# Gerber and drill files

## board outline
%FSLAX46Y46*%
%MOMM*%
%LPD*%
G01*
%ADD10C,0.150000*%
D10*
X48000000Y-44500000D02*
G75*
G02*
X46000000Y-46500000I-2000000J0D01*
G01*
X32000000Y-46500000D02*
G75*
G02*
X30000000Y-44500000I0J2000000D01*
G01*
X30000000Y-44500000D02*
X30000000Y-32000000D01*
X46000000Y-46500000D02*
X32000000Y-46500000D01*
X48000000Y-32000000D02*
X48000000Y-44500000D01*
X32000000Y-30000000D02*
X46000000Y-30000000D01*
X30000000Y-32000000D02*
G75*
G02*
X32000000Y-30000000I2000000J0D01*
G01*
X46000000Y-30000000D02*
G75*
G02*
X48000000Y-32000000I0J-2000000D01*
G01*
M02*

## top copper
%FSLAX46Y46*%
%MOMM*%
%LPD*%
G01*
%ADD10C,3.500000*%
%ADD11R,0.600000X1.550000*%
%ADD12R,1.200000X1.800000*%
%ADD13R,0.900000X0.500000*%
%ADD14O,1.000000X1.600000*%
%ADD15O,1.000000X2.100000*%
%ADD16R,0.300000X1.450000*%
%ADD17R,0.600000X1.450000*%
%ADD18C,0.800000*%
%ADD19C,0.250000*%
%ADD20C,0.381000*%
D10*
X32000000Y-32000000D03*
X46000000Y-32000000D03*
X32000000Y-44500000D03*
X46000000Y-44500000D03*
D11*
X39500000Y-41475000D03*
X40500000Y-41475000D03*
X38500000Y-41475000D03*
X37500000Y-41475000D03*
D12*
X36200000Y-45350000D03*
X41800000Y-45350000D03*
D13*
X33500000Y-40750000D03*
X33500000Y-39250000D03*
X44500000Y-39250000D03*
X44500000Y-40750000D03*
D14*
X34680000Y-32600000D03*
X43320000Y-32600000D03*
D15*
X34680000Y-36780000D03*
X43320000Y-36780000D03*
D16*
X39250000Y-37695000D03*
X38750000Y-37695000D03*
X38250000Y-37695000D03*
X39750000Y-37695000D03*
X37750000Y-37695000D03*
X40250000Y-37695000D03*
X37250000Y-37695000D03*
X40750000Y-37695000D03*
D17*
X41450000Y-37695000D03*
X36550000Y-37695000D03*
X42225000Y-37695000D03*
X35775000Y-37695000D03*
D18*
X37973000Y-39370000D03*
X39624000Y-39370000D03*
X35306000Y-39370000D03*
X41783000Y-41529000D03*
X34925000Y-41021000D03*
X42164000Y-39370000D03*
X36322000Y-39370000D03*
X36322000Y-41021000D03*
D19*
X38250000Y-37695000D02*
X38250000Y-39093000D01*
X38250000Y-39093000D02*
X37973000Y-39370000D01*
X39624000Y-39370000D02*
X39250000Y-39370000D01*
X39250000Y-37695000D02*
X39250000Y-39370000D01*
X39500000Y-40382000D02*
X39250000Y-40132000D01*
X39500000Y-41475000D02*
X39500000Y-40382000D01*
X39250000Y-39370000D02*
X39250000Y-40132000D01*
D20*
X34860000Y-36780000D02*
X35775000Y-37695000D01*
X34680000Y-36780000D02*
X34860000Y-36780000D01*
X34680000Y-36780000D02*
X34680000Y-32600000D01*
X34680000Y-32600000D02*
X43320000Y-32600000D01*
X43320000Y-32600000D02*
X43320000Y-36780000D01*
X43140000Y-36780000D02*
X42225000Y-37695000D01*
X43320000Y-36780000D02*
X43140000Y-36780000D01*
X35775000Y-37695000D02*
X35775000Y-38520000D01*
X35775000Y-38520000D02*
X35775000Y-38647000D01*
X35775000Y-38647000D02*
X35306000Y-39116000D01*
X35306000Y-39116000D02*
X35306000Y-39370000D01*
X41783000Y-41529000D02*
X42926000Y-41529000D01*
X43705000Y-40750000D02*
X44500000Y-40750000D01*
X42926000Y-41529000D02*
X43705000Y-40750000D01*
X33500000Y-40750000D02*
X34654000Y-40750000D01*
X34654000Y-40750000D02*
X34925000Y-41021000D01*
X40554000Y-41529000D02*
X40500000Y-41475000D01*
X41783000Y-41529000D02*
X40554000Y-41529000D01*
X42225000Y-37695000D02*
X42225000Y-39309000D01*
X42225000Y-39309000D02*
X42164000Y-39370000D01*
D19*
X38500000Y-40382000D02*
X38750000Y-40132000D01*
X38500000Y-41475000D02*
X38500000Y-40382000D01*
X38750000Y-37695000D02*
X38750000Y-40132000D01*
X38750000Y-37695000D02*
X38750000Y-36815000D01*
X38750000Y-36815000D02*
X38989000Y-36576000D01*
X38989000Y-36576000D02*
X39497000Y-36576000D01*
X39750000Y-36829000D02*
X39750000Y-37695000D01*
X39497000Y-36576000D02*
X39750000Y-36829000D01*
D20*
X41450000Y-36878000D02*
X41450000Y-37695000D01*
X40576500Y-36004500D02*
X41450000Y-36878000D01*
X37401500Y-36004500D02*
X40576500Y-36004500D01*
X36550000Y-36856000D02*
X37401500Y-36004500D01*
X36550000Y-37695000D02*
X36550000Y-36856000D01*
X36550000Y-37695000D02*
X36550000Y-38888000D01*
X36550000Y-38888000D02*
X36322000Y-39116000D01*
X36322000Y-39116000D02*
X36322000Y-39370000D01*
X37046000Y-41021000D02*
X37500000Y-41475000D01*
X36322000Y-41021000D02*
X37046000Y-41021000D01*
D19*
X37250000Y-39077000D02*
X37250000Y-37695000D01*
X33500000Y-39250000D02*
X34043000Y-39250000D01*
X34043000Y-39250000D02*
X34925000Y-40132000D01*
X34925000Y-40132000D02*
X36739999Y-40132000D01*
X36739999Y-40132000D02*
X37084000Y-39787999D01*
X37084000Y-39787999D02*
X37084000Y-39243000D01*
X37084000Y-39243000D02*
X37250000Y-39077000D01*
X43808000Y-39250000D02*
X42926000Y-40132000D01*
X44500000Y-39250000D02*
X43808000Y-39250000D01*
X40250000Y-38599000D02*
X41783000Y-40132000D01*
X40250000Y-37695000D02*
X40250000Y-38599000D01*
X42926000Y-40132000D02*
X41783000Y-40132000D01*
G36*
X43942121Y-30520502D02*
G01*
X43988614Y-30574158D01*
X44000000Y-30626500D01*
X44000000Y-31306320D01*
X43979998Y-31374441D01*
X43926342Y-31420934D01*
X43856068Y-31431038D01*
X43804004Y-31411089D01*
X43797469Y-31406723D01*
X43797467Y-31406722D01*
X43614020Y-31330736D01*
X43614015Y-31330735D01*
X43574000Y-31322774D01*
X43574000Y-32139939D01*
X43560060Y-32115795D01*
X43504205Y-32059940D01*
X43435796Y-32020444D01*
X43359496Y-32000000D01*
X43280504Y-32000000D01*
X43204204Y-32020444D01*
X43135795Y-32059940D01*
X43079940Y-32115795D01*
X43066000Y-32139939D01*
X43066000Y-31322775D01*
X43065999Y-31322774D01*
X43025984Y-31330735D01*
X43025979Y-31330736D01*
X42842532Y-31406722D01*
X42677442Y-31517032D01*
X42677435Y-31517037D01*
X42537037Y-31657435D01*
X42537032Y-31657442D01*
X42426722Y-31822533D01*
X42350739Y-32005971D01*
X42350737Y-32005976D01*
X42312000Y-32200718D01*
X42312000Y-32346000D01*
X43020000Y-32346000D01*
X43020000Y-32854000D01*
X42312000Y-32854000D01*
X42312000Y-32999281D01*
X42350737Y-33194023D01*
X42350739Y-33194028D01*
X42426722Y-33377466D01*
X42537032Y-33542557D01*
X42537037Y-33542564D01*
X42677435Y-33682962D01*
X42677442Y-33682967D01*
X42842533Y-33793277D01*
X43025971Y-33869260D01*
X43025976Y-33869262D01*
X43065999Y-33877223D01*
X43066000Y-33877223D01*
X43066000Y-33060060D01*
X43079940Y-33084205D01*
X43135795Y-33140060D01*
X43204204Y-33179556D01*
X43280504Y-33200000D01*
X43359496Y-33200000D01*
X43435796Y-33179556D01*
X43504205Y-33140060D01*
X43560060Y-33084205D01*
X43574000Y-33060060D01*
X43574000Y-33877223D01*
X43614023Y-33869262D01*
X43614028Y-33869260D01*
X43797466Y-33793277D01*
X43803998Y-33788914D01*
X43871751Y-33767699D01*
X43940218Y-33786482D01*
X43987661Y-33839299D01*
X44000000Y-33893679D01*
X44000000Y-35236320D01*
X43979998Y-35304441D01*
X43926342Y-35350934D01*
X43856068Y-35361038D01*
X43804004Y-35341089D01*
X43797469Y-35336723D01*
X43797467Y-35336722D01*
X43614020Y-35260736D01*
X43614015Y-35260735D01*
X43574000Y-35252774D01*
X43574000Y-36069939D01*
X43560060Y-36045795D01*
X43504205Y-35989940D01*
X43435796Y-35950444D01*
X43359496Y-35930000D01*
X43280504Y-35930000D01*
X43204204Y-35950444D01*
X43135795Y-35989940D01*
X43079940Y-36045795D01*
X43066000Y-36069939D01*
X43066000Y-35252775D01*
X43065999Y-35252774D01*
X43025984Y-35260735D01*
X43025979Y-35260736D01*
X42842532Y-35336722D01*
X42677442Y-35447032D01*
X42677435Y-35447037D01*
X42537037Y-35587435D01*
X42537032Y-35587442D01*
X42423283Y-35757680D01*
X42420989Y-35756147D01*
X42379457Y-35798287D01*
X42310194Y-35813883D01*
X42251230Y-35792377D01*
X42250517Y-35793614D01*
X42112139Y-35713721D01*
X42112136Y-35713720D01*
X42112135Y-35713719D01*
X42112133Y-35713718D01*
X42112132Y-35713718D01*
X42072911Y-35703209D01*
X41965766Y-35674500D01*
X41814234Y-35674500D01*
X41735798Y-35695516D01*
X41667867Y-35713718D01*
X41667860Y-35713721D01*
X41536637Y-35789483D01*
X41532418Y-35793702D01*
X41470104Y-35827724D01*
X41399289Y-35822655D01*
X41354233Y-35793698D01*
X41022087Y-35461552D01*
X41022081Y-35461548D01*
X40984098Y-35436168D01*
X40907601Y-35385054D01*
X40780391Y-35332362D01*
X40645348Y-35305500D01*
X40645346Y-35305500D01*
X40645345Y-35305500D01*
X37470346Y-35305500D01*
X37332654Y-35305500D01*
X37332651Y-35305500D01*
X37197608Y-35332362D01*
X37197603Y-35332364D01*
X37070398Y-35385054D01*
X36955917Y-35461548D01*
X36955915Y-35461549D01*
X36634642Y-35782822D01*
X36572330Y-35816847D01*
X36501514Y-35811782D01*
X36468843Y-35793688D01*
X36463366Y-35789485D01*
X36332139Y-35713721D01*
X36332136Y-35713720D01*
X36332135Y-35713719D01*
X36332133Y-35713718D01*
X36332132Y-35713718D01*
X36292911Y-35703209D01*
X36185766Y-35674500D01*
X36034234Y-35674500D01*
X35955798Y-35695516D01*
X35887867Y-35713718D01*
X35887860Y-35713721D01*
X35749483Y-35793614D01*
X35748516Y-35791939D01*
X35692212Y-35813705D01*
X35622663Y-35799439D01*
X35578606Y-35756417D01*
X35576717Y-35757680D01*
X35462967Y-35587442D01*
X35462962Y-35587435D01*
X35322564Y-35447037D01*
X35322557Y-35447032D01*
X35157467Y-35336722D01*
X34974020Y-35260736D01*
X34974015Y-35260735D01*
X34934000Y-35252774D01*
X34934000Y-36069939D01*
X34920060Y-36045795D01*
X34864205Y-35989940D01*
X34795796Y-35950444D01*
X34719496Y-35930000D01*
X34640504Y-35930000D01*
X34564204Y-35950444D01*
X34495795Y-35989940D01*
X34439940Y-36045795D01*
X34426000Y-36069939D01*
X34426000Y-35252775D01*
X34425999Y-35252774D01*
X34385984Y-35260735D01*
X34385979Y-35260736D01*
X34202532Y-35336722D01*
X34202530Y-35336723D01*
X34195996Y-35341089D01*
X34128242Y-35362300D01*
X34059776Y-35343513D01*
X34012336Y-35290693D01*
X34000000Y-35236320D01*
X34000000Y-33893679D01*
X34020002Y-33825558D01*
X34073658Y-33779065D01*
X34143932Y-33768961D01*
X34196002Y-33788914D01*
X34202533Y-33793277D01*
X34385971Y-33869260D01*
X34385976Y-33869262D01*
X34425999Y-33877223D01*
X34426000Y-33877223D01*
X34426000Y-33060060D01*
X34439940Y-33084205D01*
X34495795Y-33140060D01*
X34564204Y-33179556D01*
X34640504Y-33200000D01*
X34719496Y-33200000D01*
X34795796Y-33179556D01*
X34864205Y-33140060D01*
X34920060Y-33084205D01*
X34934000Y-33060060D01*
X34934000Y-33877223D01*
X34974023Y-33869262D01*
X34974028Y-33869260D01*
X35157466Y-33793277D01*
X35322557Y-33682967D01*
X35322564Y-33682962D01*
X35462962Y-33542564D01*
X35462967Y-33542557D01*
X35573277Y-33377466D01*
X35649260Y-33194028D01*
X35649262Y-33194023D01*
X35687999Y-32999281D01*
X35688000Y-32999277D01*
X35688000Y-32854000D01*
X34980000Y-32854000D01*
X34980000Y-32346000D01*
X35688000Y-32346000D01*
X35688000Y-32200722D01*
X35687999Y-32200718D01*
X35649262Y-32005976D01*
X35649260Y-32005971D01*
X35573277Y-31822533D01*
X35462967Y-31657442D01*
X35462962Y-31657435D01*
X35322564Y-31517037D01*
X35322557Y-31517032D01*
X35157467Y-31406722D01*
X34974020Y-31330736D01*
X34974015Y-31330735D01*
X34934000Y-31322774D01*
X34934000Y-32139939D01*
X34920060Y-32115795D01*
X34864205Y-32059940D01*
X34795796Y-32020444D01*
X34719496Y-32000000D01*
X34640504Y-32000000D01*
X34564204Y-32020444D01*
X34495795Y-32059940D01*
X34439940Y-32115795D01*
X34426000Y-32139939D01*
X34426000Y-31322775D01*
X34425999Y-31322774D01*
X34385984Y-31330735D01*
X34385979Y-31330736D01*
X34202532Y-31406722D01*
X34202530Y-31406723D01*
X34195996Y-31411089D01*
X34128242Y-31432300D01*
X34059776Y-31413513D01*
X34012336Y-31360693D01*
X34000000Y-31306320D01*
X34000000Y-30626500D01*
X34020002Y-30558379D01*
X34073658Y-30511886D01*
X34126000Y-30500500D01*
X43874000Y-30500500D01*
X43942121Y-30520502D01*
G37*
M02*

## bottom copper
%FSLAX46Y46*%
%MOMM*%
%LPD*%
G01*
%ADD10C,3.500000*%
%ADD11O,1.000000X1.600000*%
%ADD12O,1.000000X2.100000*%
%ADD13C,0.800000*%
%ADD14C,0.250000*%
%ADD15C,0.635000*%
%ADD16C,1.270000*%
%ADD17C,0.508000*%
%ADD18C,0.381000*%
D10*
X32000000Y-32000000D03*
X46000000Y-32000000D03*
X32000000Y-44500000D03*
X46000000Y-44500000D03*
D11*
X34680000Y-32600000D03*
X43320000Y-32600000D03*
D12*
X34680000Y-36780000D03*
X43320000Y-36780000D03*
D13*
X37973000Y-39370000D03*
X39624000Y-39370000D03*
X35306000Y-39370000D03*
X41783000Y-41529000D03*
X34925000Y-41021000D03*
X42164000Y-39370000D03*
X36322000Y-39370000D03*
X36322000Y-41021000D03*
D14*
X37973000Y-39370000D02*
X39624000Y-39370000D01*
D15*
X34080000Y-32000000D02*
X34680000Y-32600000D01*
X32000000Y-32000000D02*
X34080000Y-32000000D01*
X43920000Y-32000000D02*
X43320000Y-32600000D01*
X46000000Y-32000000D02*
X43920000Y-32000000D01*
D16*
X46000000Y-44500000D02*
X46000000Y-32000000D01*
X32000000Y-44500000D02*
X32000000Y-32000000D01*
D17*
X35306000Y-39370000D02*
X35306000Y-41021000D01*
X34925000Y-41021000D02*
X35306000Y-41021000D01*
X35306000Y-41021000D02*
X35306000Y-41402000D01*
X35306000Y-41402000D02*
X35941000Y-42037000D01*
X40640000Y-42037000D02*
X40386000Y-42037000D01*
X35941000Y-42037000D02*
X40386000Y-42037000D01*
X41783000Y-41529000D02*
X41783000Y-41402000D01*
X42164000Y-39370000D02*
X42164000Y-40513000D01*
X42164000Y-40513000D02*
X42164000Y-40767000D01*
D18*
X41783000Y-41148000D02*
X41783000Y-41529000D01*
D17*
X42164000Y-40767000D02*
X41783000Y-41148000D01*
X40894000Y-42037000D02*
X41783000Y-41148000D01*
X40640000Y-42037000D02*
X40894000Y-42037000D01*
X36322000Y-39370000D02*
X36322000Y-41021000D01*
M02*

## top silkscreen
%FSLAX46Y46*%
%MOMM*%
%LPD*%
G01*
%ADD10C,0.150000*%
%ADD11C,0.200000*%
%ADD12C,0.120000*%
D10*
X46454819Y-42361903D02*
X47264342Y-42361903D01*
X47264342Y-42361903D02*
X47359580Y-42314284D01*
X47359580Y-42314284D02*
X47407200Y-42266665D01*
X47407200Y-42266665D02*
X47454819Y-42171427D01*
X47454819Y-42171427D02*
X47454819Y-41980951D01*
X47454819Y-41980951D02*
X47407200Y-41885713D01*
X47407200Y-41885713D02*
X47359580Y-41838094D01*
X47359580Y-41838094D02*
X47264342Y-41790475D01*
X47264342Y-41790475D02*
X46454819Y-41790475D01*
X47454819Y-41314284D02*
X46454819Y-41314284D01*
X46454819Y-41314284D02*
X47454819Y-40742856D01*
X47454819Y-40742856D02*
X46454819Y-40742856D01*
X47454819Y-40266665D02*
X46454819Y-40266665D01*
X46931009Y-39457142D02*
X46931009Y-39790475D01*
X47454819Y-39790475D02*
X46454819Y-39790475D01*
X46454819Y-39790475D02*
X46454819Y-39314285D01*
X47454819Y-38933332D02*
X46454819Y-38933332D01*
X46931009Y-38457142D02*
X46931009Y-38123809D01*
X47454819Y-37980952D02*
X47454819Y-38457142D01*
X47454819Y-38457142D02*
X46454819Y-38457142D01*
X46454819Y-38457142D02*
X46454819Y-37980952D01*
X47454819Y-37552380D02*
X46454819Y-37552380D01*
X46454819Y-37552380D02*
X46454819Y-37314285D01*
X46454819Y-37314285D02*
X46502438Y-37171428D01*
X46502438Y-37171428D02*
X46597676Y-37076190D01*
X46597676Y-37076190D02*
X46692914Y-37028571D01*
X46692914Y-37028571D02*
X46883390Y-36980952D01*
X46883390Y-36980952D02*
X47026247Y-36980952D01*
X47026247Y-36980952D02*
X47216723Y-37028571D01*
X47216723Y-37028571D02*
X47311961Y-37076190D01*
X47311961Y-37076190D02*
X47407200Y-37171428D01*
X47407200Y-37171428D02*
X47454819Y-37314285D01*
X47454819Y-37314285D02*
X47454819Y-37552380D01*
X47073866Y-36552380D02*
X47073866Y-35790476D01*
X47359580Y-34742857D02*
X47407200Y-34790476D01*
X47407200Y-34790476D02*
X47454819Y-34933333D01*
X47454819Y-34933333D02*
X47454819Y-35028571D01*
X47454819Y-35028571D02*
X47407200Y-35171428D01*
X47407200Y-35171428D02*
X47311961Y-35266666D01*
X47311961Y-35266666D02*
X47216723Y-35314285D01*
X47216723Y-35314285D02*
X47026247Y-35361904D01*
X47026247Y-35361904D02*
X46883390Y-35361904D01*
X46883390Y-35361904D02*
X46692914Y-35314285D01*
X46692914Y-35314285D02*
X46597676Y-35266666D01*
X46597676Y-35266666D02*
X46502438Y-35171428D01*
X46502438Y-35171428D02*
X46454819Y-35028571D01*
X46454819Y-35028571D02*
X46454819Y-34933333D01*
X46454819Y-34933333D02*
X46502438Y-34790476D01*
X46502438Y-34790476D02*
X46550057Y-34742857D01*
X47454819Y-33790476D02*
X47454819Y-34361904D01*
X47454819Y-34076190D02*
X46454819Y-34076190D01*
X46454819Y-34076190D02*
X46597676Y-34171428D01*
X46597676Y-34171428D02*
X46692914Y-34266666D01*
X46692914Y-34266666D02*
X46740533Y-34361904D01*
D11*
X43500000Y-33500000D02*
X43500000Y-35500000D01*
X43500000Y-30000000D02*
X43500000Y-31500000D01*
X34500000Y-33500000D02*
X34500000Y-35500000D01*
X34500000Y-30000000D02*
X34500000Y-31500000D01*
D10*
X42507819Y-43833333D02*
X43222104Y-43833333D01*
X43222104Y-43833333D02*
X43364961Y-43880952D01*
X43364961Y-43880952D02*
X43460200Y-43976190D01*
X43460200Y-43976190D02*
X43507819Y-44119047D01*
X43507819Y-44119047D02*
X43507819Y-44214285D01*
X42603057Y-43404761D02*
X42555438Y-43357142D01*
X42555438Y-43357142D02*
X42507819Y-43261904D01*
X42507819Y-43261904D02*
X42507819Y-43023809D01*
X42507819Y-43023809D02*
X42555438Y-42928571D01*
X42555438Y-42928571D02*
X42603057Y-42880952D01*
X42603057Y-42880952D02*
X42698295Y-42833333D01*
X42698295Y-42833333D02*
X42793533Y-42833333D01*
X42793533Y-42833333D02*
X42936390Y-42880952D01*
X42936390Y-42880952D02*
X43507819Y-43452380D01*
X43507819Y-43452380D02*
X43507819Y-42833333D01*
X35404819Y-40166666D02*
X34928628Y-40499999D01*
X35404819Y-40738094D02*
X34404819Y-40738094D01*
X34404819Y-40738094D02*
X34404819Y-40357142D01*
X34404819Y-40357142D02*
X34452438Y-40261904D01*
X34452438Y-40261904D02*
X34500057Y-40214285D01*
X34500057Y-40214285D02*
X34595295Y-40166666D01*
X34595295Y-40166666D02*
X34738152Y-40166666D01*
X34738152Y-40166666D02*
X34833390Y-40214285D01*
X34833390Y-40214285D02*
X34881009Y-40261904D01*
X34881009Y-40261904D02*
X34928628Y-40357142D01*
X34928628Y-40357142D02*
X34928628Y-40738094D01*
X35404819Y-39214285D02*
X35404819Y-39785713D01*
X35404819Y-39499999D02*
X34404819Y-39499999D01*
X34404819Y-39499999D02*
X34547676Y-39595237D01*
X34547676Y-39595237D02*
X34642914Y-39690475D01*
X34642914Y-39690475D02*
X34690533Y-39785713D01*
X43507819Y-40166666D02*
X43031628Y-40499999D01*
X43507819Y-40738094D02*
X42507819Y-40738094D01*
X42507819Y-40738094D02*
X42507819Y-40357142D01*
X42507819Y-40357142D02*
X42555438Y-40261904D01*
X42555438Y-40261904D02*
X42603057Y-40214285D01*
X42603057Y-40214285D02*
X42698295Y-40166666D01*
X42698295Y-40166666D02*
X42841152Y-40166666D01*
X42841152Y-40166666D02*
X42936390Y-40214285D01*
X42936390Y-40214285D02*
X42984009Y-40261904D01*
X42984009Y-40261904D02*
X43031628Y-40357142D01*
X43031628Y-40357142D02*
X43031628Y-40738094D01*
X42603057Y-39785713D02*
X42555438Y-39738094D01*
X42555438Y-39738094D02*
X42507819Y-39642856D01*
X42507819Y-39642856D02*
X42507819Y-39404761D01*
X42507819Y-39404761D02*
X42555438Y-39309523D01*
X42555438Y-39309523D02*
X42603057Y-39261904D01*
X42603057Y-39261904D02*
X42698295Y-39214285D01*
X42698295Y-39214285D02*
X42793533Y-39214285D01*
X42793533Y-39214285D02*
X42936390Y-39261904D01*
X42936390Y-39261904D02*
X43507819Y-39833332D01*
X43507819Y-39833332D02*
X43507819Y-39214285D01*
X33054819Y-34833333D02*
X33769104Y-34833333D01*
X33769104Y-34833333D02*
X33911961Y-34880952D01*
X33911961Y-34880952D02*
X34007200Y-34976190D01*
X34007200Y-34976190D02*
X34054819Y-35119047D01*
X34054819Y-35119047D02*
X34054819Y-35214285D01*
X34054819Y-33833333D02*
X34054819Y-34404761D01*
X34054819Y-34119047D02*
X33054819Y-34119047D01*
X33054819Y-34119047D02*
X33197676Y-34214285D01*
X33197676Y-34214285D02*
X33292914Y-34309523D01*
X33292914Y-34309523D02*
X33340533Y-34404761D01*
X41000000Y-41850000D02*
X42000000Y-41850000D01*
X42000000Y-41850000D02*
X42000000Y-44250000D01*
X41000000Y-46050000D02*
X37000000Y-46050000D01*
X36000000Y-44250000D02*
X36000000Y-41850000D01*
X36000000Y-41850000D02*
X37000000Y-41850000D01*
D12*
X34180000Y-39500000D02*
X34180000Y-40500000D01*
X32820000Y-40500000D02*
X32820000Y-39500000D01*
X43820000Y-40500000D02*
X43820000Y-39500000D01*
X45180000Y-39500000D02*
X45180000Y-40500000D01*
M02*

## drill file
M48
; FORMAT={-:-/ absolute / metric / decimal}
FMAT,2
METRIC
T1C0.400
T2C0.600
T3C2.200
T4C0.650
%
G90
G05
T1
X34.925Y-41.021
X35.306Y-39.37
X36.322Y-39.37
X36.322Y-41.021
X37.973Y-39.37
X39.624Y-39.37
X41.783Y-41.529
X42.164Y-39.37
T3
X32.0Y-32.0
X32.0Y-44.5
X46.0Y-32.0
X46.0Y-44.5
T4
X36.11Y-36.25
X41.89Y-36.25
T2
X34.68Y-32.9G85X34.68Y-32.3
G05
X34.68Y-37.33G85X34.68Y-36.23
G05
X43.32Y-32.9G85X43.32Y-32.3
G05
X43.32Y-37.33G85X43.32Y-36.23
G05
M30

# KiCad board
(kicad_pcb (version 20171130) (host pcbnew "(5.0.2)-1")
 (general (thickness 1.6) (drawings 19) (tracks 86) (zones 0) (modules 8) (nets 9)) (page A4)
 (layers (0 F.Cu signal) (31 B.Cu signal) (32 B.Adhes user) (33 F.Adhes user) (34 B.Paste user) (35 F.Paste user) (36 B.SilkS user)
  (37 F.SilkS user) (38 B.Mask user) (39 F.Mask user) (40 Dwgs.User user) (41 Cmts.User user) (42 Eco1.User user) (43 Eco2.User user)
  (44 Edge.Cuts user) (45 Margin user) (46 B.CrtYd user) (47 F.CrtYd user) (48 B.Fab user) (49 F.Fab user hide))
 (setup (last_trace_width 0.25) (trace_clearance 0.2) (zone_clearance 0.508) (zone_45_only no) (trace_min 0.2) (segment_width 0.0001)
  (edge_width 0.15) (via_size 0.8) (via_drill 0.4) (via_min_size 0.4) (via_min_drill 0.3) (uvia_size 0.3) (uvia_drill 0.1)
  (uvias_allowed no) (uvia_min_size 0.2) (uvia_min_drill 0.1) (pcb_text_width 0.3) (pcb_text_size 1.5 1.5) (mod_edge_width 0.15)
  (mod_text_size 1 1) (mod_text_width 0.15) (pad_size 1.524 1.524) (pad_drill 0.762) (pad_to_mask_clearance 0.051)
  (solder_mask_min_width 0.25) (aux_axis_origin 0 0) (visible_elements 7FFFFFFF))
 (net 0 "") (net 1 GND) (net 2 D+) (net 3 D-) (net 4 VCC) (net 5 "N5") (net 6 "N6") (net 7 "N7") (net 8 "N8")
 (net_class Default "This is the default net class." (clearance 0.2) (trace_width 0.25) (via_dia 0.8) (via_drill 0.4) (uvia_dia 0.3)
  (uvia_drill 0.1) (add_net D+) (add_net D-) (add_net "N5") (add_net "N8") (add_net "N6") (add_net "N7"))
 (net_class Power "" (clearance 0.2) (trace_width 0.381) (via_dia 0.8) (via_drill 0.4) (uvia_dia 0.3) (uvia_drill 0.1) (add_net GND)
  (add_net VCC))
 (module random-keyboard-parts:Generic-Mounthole (layer F.Cu) (at 32 32)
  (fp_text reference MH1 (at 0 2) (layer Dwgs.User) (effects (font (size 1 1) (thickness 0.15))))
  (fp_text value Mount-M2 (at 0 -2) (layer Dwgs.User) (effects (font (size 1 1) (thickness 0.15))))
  (pad 1 thru_hole circle (at 0 0) (size 3.5 3.5) (drill 2.2) (layers *.Cu *.Mask) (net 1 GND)))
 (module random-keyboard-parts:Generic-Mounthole (layer F.Cu) (at 46 32)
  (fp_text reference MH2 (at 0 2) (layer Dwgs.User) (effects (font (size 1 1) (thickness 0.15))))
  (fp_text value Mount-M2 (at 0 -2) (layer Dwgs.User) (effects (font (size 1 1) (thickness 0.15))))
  (pad 1 thru_hole circle (at 0 0) (size 3.5 3.5) (drill 2.2) (layers *.Cu *.Mask) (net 1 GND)))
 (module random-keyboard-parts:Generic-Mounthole (layer F.Cu) (at 32 44.5)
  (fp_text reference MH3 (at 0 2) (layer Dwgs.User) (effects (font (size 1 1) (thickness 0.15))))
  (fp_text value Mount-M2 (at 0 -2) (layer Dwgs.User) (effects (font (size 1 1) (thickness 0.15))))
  (pad 1 thru_hole circle (at 0 0) (size 3.5 3.5) (drill 2.2) (layers *.Cu *.Mask) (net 1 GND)))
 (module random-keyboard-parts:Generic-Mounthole (layer F.Cu) (at 46 44.5)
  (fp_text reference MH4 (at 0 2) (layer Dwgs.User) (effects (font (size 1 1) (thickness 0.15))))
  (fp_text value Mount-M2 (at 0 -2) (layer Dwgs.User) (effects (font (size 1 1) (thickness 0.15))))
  (pad 1 thru_hole circle (at 0 0) (size 3.5 3.5) (drill 2.2) (layers *.Cu *.Mask) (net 1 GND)))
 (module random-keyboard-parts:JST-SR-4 (layer F.Cu) (at 39 46.25)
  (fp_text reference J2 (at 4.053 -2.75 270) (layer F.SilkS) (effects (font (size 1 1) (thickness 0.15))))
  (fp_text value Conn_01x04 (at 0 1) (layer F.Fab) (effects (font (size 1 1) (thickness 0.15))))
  (fp_line (start 2 -4.4) (end 3 -4.4) (layer F.SilkS) (width 0.15))
  (fp_line (start 3 -4.4) (end 3 -2) (layer F.SilkS) (width 0.15))
  (fp_line (start 2 -0.2) (end -2 -0.2) (layer F.SilkS) (width 0.15))
  (fp_line (start -3 -2) (end -3 -4.4) (layer F.SilkS) (width 0.15))
  (fp_line (start -3 -4.4) (end -2 -4.4) (layer F.SilkS) (width 0.15))
  (pad 3 smd rect (at 0.5 -4.775) (size 0.6 1.55) (layers F.Cu F.Paste F.Mask) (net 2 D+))
  (pad 4 smd rect (at 1.5 -4.775) (size 0.6 1.55) (layers F.Cu F.Paste F.Mask) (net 1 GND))
  (pad 2 smd rect (at -0.5 -4.775) (size 0.6 1.55) (layers F.Cu F.Paste F.Mask) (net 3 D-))
  (pad 1 smd rect (at -1.5 -4.775) (size 0.6 1.55) (layers F.Cu F.Paste F.Mask) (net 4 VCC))
  (pad "" smd rect (at -2.8 -0.9) (size 1.2 1.8) (layers F.Cu F.Paste F.Mask))
  (pad "" smd rect (at 2.8 -0.9) (size 1.2 1.8) (layers F.Cu F.Paste F.Mask)))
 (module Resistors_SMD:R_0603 (layer F.Cu) (at 33.5 40 270)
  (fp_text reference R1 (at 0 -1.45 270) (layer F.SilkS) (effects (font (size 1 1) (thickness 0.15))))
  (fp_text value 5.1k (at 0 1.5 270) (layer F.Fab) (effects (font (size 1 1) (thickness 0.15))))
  (fp_line (start -0.5 -0.68) (end 0.5 -0.68) (layer F.SilkS) (width 0.12))
  (fp_line (start 0.5 0.68) (end -0.5 0.68) (layer F.SilkS) (width 0.12))
  (pad 2 smd rect (at 0.75 0 270) (size 0.5 0.9) (layers F.Cu F.Paste F.Mask) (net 1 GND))
  (pad 1 smd rect (at -0.75 0 270) (size 0.5 0.9) (layers F.Cu F.Paste F.Mask) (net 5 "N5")))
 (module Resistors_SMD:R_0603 (layer F.Cu) (at 44.5 40 270)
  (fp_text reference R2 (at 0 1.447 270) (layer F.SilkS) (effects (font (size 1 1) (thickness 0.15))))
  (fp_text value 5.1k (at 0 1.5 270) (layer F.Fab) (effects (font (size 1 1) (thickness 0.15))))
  (fp_line (start 0.5 0.68) (end -0.5 0.68) (layer F.SilkS) (width 0.12))
  (fp_line (start -0.5 -0.68) (end 0.5 -0.68) (layer F.SilkS) (width 0.12))
  (pad 1 smd rect (at -0.75 0 270) (size 0.5 0.9) (layers F.Cu F.Paste F.Mask) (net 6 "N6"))
  (pad 2 smd rect (at 0.75 0 270) (size 0.5 0.9) (layers F.Cu F.Paste F.Mask) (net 1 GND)))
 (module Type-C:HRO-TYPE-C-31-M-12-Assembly (layer F.Cu) (at 39 30 180)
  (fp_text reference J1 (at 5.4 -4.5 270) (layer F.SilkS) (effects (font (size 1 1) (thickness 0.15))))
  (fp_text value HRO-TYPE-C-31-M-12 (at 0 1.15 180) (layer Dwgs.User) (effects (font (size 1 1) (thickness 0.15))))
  (pad 13 thru_hole oval (at 4.32 -2.6 180) (size 1 1.6) (drill oval 0.6 1.2) (layers *.Cu *.Mask) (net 1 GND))
  (pad 13 thru_hole oval (at -4.32 -2.6 180) (size 1 1.6) (drill oval 0.6 1.2) (layers *.Cu *.Mask) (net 1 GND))
  (pad 13 thru_hole oval (at 4.32 -6.78 180) (size 1 2.1) (drill oval 0.6 1.7) (layers *.Cu *.Mask) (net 1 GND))
  (pad 13 thru_hole oval (at -4.32 -6.78 180) (size 1 2.1) (drill oval 0.6 1.7) (layers *.Cu *.Mask) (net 1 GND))
  (pad "" np_thru_hole circle (at -2.89 -6.25 180) (size 0.65 0.65) (drill 0.65) (layers *.Cu *.Mask))
  (pad "" np_thru_hole circle (at 2.89 -6.25 180) (size 0.65 0.65) (drill 0.65) (layers *.Cu *.Mask))
  (pad 6 smd rect (at -0.25 -7.695 180) (size 0.3 1.45) (layers F.Cu F.Paste F.Mask) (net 2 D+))
  (pad 7 smd rect (at 0.25 -7.695 180) (size 0.3 1.45) (layers F.Cu F.Paste F.Mask) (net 3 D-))
  (pad 8 smd rect (at 0.75 -7.695 180) (size 0.3 1.45) (layers F.Cu F.Paste F.Mask) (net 2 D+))
  (pad 5 smd rect (at -0.75 -7.695 180) (size 0.3 1.45) (layers F.Cu F.Paste F.Mask) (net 3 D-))
  (pad 9 smd rect (at 1.25 -7.695 180) (size 0.3 1.45) (layers F.Cu F.Paste F.Mask) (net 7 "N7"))
  (pad 4 smd rect (at -1.25 -7.695 180) (size 0.3 1.45) (layers F.Cu F.Paste F.Mask) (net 6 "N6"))
  (pad 10 smd rect (at 1.75 -7.695 180) (size 0.3 1.45) (layers F.Cu F.Paste F.Mask) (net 5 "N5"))
  (pad 3 smd rect (at -1.75 -7.695 180) (size 0.3 1.45) (layers F.Cu F.Paste F.Mask) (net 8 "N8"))
  (pad 2 smd rect (at -2.45 -7.695 180) (size 0.6 1.45) (layers F.Cu F.Paste F.Mask) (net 4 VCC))
  (pad 11 smd rect (at 2.45 -7.695 180) (size 0.6 1.45) (layers F.Cu F.Paste F.Mask) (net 4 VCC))
  (pad 1 smd rect (at -3.225 -7.695 180) (size 0.6 1.45) (layers F.Cu F.Paste F.Mask) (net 1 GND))
  (pad 12 smd rect (at 3.225 -7.695 180) (size 0.6 1.45) (layers F.Cu F.Paste F.Mask) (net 1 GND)))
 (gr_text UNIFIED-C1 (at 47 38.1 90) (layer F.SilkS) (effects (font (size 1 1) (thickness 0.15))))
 (gr_line (start 43.5 33.5) (end 43.5 35.5) (layer F.SilkS) (width 0.2))
 (gr_line (start 43.5 30) (end 43.5 31.5) (layer F.SilkS) (width 0.2))
 (gr_line (start 34.5 33.5) (end 34.5 35.5) (layer F.SilkS) (width 0.2))
 (gr_line (start 34.5 30) (end 34.5 31.5) (layer F.SilkS) (width 0.2))
 (gr_arc (start 46 44.5) (end 46 46.5) (angle -90) (layer Edge.Cuts) (width 0.15))
 (gr_arc (start 32 44.5) (end 30 44.5) (angle -90) (layer Edge.Cuts) (width 0.15))
 (gr_line (start 30 44.5) (end 30 32) (layer Edge.Cuts) (width 0.15))
 (gr_line (start 46 46.5) (end 32 46.5) (layer Edge.Cuts) (width 0.15))
 (gr_line (start 48 32) (end 48 44.5) (layer Edge.Cuts) (width 0.15))
 (gr_line (start 32 30) (end 46 30) (layer Edge.Cuts) (width 0.15))
 (gr_arc (start 32 32) (end 32 30) (angle -90) (layer Edge.Cuts) (width 0.15))
 (gr_arc (start 46 32) (end 48 32) (angle -90) (layer Edge.Cuts) (width 0.15))
 (via (at 37.973 39.37) (size 0.8) (drill 0.4) (layers F.Cu B.Cu) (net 2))
 (segment (start 38.25 37.695) (end 38.25 39.093) (width 0.25) (layer F.Cu) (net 2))
 (segment (start 38.25 39.093) (end 37.973 39.37) (width 0.25) (layer F.Cu) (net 2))
 (via (at 39.624 39.37) (size 0.8) (drill 0.4) (layers F.Cu B.Cu) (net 2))
 (segment (start 37.973 39.37) (end 39.624 39.37) (width 0.25) (layer B.Cu) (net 2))
 (segment (start 39.624 39.37) (end 39.25 39.37) (width 0.25) (layer F.Cu) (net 2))
 (segment (start 39.25 37.695) (end 39.25 39.37) (width 0.25) (layer F.Cu) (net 2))
 (segment (start 39.5 40.382) (end 39.25 40.132) (width 0.25) (layer F.Cu) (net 2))
 (segment (start 39.5 41.475) (end 39.5 40.382) (width 0.25) (layer F.Cu) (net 2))
 (segment (start 39.25 39.37) (end 39.25 40.132) (width 0.25) (layer F.Cu) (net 2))
 (segment (start 34.86 36.78) (end 35.775 37.695) (width 0.381) (layer F.Cu) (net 1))
 (segment (start 34.68 36.78) (end 34.86 36.78) (width 0.381) (layer F.Cu) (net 1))
 (segment (start 34.68 36.78) (end 34.68 32.6) (width 0.381) (layer F.Cu) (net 1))
 (segment (start 34.68 32.6) (end 43.32 32.6) (width 0.381) (layer F.Cu) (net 1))
 (segment (start 43.32 32.6) (end 43.32 36.78) (width 0.381) (layer F.Cu) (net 1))
 (segment (start 43.14 36.78) (end 42.225 37.695) (width 0.381) (layer F.Cu) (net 1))
 (segment (start 43.32 36.78) (end 43.14 36.78) (width 0.381) (layer F.Cu) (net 1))
 (segment (start 35.775 37.695) (end 35.775 38.52) (width 0.381) (layer F.Cu) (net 1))
 (segment (start 35.775 38.52) (end 35.775 38.647) (width 0.381) (layer F.Cu) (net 1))
 (via (at 35.306 39.37) (size 0.8) (drill 0.4) (layers F.Cu B.Cu) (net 1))
 (segment (start 35.775 38.647) (end 35.306 39.116) (width 0.381) (layer F.Cu) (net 1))
 (segment (start 35.306 39.116) (end 35.306 39.37) (width 0.381) (layer F.Cu) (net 1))
 (via (at 41.783 41.529) (size 0.8) (drill 0.4) (layers F.Cu B.Cu) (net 1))
 (segment (start 41.783 41.529) (end 42.926 41.529) (width 0.381) (layer F.Cu) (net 1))
 (segment (start 43.705 40.75) (end 44.5 40.75) (width 0.381) (layer F.Cu) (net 1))
 (segment (start 42.926 41.529) (end 43.705 40.75) (width 0.381) (layer F.Cu) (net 1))
 (via (at 34.925 41.021) (size 0.8) (drill 0.4) (layers F.Cu B.Cu) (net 1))
 (segment (start 33.5 40.75) (end 34.654 40.75) (width 0.381) (layer F.Cu) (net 1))
 (segment (start 34.654 40.75) (end 34.925 41.021) (width 0.381) (layer F.Cu) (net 1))
 (segment (start 34.08 32) (end 34.68 32.6) (width 0.635) (layer B.Cu) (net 1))
 (segment (start 32 32) (end 34.08 32) (width 0.635) (layer B.Cu) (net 1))
 (segment (start 40.554 41.529) (end 40.5 41.475) (width 0.381) (layer F.Cu) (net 1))
 (segment (start 41.783 41.529) (end 40.554 41.529) (width 0.381) (layer F.Cu) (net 1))
 (segment (start 43.92 32) (end 43.32 32.6) (width 0.635) (layer B.Cu) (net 1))
 (segment (start 46 32) (end 43.92 32) (width 0.635) (layer B.Cu) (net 1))
 (segment (start 46 44.5) (end 46 32) (width 1.27) (layer B.Cu) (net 1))
 (segment (start 32 44.5) (end 32 32) (width 1.27) (layer B.Cu) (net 1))
 (segment (start 35.306 39.37) (end 35.306 41.021) (width 0.508) (layer B.Cu) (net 1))
 (segment (start 34.925 41.021) (end 35.306 41.021) (width 0.508) (layer B.Cu) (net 1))
 (segment (start 35.306 41.021) (end 35.306 41.402) (width 0.508) (layer B.Cu) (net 1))
 (segment (start 35.306 41.402) (end 35.941 42.037) (width 0.508) (layer B.Cu) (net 1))
 (segment (start 40.64 42.037) (end 40.386 42.037) (width 0.508) (layer B.Cu) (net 1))
 (segment (start 35.941 42.037) (end 40.386 42.037) (width 0.508) (layer B.Cu) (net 1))
 (segment (start 41.783 41.529) (end 41.783 41.402) (width 0.508) (layer B.Cu) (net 1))
 (via (at 42.164 39.37) (size 0.8) (drill 0.4) (layers F.Cu B.Cu) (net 1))
 (segment (start 42.225 37.695) (end 42.225 39.309) (width 0.381) (layer F.Cu) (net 1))
 (segment (start 42.225 39.309) (end 42.164 39.37) (width 0.381) (layer F.Cu) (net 1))
 (segment (start 42.164 39.37) (end 42.164 40.513) (width 0.508) (layer B.Cu) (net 1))
 (segment (start 42.164 40.513) (end 42.164 40.767) (width 0.508) (layer B.Cu) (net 1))
 (segment (start 41.783 41.148) (end 41.783 41.529) (width 0.381) (layer B.Cu) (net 1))
 (segment (start 42.164 40.767) (end 41.783 41.148) (width 0.508) (layer B.Cu) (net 1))
 (segment (start 40.894 42.037) (end 41.783 41.148) (width 0.508) (layer B.Cu) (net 1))
 (segment (start 40.64 42.037) (end 40.894 42.037) (width 0.508) (layer B.Cu) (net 1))
 (segment (start 38.5 40.382) (end 38.75 40.132) (width 0.25) (layer F.Cu) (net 3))
 (segment (start 38.5 41.475) (end 38.5 40.382) (width 0.25) (layer F.Cu) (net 3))
 (segment (start 38.75 37.695) (end 38.75 40.132) (width 0.25) (layer F.Cu) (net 3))
 (segment (start 38.75 37.695) (end 38.75 36.815) (width 0.25) (layer F.Cu) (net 3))
 (segment (start 38.75 36.815) (end 38.989 36.576) (width 0.25) (layer F.Cu) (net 3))
 (segment (start 38.989 36.576) (end 39.497 36.576) (width 0.25) (layer F.Cu) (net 3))
 (segment (start 39.75 36.829) (end 39.75 37.695) (width 0.25) (layer F.Cu) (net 3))
 (segment (start 39.497 36.576) (end 39.75 36.829) (width 0.25) (layer F.Cu) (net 3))
 (segment (start 41.45 36.878) (end 41.45 37.695) (width 0.381) (layer F.Cu) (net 4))
 (segment (start 40.5765 36.0045) (end 41.45 36.878) (width 0.381) (layer F.Cu) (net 4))
 (segment (start 37.4015 36.0045) (end 40.5765 36.0045) (width 0.381) (layer F.Cu) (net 4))
 (segment (start 36.55 36.856) (end 37.4015 36.0045) (width 0.381) (layer F.Cu) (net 4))
 (segment (start 36.55 37.695) (end 36.55 36.856) (width 0.381) (layer F.Cu) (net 4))
 (segment (start 36.55 37.695) (end 36.55 38.888) (width 0.381) (layer F.Cu) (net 4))
 (segment (start 36.55 38.888) (end 36.322 39.116) (width 0.381) (layer F.Cu) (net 4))
 (segment (start 36.322 39.116) (end 36.322 39.37) (width 0.381) (layer F.Cu) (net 4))
 (via (at 36.322 39.37) (size 0.8) (drill 0.4) (layers F.Cu B.Cu) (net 4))
 (via (at 36.322 41.021) (size 0.8) (drill 0.4) (layers F.Cu B.Cu) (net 4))
 (segment (start 37.046 41.021) (end 37.5 41.475) (width 0.381) (layer F.Cu) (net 4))
 (segment (start 36.322 41.021) (end 37.046 41.021) (width 0.381) (layer F.Cu) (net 4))
 (segment (start 36.322 39.37) (end 36.322 41.021) (width 0.508) (layer B.Cu) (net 4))
 (segment (start 37.25 39.077) (end 37.25 37.695) (width 0.25) (layer F.Cu) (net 5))
 (segment (start 33.5 39.25) (end 34.043 39.25) (width 0.25) (layer F.Cu) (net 5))
 (segment (start 34.043 39.25) (end 34.925 40.132) (width 0.25) (layer F.Cu) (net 5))
 (segment (start 34.925 40.132) (end 36.739999 40.132) (width 0.25) (layer F.Cu) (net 5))
 (segment (start 36.739999 40.132) (end 37.084 39.787999) (width 0.25) (layer F.Cu) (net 5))
 (segment (start 37.084 39.787999) (end 37.084 39.243) (width 0.25) (layer F.Cu) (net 5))
 (segment (start 37.084 39.243) (end 37.25 39.077) (width 0.25) (layer F.Cu) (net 5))
 (segment (start 43.808 39.25) (end 42.926 40.132) (width 0.25) (layer F.Cu) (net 6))
 (segment (start 44.5 39.25) (end 43.808 39.25) (width 0.25) (layer F.Cu) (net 6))
 (segment (start 40.25 38.599) (end 41.783 40.132) (width 0.25) (layer F.Cu) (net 6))
 (segment (start 40.25 37.695) (end 40.25 38.599) (width 0.25) (layer F.Cu) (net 6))
 (segment (start 42.926 40.132) (end 41.783 40.132) (width 0.25) (layer F.Cu) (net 6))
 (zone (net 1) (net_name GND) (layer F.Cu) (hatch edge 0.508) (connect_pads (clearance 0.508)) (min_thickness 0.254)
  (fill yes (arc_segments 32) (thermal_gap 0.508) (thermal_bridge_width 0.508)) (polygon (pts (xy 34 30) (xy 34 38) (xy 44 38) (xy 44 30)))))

